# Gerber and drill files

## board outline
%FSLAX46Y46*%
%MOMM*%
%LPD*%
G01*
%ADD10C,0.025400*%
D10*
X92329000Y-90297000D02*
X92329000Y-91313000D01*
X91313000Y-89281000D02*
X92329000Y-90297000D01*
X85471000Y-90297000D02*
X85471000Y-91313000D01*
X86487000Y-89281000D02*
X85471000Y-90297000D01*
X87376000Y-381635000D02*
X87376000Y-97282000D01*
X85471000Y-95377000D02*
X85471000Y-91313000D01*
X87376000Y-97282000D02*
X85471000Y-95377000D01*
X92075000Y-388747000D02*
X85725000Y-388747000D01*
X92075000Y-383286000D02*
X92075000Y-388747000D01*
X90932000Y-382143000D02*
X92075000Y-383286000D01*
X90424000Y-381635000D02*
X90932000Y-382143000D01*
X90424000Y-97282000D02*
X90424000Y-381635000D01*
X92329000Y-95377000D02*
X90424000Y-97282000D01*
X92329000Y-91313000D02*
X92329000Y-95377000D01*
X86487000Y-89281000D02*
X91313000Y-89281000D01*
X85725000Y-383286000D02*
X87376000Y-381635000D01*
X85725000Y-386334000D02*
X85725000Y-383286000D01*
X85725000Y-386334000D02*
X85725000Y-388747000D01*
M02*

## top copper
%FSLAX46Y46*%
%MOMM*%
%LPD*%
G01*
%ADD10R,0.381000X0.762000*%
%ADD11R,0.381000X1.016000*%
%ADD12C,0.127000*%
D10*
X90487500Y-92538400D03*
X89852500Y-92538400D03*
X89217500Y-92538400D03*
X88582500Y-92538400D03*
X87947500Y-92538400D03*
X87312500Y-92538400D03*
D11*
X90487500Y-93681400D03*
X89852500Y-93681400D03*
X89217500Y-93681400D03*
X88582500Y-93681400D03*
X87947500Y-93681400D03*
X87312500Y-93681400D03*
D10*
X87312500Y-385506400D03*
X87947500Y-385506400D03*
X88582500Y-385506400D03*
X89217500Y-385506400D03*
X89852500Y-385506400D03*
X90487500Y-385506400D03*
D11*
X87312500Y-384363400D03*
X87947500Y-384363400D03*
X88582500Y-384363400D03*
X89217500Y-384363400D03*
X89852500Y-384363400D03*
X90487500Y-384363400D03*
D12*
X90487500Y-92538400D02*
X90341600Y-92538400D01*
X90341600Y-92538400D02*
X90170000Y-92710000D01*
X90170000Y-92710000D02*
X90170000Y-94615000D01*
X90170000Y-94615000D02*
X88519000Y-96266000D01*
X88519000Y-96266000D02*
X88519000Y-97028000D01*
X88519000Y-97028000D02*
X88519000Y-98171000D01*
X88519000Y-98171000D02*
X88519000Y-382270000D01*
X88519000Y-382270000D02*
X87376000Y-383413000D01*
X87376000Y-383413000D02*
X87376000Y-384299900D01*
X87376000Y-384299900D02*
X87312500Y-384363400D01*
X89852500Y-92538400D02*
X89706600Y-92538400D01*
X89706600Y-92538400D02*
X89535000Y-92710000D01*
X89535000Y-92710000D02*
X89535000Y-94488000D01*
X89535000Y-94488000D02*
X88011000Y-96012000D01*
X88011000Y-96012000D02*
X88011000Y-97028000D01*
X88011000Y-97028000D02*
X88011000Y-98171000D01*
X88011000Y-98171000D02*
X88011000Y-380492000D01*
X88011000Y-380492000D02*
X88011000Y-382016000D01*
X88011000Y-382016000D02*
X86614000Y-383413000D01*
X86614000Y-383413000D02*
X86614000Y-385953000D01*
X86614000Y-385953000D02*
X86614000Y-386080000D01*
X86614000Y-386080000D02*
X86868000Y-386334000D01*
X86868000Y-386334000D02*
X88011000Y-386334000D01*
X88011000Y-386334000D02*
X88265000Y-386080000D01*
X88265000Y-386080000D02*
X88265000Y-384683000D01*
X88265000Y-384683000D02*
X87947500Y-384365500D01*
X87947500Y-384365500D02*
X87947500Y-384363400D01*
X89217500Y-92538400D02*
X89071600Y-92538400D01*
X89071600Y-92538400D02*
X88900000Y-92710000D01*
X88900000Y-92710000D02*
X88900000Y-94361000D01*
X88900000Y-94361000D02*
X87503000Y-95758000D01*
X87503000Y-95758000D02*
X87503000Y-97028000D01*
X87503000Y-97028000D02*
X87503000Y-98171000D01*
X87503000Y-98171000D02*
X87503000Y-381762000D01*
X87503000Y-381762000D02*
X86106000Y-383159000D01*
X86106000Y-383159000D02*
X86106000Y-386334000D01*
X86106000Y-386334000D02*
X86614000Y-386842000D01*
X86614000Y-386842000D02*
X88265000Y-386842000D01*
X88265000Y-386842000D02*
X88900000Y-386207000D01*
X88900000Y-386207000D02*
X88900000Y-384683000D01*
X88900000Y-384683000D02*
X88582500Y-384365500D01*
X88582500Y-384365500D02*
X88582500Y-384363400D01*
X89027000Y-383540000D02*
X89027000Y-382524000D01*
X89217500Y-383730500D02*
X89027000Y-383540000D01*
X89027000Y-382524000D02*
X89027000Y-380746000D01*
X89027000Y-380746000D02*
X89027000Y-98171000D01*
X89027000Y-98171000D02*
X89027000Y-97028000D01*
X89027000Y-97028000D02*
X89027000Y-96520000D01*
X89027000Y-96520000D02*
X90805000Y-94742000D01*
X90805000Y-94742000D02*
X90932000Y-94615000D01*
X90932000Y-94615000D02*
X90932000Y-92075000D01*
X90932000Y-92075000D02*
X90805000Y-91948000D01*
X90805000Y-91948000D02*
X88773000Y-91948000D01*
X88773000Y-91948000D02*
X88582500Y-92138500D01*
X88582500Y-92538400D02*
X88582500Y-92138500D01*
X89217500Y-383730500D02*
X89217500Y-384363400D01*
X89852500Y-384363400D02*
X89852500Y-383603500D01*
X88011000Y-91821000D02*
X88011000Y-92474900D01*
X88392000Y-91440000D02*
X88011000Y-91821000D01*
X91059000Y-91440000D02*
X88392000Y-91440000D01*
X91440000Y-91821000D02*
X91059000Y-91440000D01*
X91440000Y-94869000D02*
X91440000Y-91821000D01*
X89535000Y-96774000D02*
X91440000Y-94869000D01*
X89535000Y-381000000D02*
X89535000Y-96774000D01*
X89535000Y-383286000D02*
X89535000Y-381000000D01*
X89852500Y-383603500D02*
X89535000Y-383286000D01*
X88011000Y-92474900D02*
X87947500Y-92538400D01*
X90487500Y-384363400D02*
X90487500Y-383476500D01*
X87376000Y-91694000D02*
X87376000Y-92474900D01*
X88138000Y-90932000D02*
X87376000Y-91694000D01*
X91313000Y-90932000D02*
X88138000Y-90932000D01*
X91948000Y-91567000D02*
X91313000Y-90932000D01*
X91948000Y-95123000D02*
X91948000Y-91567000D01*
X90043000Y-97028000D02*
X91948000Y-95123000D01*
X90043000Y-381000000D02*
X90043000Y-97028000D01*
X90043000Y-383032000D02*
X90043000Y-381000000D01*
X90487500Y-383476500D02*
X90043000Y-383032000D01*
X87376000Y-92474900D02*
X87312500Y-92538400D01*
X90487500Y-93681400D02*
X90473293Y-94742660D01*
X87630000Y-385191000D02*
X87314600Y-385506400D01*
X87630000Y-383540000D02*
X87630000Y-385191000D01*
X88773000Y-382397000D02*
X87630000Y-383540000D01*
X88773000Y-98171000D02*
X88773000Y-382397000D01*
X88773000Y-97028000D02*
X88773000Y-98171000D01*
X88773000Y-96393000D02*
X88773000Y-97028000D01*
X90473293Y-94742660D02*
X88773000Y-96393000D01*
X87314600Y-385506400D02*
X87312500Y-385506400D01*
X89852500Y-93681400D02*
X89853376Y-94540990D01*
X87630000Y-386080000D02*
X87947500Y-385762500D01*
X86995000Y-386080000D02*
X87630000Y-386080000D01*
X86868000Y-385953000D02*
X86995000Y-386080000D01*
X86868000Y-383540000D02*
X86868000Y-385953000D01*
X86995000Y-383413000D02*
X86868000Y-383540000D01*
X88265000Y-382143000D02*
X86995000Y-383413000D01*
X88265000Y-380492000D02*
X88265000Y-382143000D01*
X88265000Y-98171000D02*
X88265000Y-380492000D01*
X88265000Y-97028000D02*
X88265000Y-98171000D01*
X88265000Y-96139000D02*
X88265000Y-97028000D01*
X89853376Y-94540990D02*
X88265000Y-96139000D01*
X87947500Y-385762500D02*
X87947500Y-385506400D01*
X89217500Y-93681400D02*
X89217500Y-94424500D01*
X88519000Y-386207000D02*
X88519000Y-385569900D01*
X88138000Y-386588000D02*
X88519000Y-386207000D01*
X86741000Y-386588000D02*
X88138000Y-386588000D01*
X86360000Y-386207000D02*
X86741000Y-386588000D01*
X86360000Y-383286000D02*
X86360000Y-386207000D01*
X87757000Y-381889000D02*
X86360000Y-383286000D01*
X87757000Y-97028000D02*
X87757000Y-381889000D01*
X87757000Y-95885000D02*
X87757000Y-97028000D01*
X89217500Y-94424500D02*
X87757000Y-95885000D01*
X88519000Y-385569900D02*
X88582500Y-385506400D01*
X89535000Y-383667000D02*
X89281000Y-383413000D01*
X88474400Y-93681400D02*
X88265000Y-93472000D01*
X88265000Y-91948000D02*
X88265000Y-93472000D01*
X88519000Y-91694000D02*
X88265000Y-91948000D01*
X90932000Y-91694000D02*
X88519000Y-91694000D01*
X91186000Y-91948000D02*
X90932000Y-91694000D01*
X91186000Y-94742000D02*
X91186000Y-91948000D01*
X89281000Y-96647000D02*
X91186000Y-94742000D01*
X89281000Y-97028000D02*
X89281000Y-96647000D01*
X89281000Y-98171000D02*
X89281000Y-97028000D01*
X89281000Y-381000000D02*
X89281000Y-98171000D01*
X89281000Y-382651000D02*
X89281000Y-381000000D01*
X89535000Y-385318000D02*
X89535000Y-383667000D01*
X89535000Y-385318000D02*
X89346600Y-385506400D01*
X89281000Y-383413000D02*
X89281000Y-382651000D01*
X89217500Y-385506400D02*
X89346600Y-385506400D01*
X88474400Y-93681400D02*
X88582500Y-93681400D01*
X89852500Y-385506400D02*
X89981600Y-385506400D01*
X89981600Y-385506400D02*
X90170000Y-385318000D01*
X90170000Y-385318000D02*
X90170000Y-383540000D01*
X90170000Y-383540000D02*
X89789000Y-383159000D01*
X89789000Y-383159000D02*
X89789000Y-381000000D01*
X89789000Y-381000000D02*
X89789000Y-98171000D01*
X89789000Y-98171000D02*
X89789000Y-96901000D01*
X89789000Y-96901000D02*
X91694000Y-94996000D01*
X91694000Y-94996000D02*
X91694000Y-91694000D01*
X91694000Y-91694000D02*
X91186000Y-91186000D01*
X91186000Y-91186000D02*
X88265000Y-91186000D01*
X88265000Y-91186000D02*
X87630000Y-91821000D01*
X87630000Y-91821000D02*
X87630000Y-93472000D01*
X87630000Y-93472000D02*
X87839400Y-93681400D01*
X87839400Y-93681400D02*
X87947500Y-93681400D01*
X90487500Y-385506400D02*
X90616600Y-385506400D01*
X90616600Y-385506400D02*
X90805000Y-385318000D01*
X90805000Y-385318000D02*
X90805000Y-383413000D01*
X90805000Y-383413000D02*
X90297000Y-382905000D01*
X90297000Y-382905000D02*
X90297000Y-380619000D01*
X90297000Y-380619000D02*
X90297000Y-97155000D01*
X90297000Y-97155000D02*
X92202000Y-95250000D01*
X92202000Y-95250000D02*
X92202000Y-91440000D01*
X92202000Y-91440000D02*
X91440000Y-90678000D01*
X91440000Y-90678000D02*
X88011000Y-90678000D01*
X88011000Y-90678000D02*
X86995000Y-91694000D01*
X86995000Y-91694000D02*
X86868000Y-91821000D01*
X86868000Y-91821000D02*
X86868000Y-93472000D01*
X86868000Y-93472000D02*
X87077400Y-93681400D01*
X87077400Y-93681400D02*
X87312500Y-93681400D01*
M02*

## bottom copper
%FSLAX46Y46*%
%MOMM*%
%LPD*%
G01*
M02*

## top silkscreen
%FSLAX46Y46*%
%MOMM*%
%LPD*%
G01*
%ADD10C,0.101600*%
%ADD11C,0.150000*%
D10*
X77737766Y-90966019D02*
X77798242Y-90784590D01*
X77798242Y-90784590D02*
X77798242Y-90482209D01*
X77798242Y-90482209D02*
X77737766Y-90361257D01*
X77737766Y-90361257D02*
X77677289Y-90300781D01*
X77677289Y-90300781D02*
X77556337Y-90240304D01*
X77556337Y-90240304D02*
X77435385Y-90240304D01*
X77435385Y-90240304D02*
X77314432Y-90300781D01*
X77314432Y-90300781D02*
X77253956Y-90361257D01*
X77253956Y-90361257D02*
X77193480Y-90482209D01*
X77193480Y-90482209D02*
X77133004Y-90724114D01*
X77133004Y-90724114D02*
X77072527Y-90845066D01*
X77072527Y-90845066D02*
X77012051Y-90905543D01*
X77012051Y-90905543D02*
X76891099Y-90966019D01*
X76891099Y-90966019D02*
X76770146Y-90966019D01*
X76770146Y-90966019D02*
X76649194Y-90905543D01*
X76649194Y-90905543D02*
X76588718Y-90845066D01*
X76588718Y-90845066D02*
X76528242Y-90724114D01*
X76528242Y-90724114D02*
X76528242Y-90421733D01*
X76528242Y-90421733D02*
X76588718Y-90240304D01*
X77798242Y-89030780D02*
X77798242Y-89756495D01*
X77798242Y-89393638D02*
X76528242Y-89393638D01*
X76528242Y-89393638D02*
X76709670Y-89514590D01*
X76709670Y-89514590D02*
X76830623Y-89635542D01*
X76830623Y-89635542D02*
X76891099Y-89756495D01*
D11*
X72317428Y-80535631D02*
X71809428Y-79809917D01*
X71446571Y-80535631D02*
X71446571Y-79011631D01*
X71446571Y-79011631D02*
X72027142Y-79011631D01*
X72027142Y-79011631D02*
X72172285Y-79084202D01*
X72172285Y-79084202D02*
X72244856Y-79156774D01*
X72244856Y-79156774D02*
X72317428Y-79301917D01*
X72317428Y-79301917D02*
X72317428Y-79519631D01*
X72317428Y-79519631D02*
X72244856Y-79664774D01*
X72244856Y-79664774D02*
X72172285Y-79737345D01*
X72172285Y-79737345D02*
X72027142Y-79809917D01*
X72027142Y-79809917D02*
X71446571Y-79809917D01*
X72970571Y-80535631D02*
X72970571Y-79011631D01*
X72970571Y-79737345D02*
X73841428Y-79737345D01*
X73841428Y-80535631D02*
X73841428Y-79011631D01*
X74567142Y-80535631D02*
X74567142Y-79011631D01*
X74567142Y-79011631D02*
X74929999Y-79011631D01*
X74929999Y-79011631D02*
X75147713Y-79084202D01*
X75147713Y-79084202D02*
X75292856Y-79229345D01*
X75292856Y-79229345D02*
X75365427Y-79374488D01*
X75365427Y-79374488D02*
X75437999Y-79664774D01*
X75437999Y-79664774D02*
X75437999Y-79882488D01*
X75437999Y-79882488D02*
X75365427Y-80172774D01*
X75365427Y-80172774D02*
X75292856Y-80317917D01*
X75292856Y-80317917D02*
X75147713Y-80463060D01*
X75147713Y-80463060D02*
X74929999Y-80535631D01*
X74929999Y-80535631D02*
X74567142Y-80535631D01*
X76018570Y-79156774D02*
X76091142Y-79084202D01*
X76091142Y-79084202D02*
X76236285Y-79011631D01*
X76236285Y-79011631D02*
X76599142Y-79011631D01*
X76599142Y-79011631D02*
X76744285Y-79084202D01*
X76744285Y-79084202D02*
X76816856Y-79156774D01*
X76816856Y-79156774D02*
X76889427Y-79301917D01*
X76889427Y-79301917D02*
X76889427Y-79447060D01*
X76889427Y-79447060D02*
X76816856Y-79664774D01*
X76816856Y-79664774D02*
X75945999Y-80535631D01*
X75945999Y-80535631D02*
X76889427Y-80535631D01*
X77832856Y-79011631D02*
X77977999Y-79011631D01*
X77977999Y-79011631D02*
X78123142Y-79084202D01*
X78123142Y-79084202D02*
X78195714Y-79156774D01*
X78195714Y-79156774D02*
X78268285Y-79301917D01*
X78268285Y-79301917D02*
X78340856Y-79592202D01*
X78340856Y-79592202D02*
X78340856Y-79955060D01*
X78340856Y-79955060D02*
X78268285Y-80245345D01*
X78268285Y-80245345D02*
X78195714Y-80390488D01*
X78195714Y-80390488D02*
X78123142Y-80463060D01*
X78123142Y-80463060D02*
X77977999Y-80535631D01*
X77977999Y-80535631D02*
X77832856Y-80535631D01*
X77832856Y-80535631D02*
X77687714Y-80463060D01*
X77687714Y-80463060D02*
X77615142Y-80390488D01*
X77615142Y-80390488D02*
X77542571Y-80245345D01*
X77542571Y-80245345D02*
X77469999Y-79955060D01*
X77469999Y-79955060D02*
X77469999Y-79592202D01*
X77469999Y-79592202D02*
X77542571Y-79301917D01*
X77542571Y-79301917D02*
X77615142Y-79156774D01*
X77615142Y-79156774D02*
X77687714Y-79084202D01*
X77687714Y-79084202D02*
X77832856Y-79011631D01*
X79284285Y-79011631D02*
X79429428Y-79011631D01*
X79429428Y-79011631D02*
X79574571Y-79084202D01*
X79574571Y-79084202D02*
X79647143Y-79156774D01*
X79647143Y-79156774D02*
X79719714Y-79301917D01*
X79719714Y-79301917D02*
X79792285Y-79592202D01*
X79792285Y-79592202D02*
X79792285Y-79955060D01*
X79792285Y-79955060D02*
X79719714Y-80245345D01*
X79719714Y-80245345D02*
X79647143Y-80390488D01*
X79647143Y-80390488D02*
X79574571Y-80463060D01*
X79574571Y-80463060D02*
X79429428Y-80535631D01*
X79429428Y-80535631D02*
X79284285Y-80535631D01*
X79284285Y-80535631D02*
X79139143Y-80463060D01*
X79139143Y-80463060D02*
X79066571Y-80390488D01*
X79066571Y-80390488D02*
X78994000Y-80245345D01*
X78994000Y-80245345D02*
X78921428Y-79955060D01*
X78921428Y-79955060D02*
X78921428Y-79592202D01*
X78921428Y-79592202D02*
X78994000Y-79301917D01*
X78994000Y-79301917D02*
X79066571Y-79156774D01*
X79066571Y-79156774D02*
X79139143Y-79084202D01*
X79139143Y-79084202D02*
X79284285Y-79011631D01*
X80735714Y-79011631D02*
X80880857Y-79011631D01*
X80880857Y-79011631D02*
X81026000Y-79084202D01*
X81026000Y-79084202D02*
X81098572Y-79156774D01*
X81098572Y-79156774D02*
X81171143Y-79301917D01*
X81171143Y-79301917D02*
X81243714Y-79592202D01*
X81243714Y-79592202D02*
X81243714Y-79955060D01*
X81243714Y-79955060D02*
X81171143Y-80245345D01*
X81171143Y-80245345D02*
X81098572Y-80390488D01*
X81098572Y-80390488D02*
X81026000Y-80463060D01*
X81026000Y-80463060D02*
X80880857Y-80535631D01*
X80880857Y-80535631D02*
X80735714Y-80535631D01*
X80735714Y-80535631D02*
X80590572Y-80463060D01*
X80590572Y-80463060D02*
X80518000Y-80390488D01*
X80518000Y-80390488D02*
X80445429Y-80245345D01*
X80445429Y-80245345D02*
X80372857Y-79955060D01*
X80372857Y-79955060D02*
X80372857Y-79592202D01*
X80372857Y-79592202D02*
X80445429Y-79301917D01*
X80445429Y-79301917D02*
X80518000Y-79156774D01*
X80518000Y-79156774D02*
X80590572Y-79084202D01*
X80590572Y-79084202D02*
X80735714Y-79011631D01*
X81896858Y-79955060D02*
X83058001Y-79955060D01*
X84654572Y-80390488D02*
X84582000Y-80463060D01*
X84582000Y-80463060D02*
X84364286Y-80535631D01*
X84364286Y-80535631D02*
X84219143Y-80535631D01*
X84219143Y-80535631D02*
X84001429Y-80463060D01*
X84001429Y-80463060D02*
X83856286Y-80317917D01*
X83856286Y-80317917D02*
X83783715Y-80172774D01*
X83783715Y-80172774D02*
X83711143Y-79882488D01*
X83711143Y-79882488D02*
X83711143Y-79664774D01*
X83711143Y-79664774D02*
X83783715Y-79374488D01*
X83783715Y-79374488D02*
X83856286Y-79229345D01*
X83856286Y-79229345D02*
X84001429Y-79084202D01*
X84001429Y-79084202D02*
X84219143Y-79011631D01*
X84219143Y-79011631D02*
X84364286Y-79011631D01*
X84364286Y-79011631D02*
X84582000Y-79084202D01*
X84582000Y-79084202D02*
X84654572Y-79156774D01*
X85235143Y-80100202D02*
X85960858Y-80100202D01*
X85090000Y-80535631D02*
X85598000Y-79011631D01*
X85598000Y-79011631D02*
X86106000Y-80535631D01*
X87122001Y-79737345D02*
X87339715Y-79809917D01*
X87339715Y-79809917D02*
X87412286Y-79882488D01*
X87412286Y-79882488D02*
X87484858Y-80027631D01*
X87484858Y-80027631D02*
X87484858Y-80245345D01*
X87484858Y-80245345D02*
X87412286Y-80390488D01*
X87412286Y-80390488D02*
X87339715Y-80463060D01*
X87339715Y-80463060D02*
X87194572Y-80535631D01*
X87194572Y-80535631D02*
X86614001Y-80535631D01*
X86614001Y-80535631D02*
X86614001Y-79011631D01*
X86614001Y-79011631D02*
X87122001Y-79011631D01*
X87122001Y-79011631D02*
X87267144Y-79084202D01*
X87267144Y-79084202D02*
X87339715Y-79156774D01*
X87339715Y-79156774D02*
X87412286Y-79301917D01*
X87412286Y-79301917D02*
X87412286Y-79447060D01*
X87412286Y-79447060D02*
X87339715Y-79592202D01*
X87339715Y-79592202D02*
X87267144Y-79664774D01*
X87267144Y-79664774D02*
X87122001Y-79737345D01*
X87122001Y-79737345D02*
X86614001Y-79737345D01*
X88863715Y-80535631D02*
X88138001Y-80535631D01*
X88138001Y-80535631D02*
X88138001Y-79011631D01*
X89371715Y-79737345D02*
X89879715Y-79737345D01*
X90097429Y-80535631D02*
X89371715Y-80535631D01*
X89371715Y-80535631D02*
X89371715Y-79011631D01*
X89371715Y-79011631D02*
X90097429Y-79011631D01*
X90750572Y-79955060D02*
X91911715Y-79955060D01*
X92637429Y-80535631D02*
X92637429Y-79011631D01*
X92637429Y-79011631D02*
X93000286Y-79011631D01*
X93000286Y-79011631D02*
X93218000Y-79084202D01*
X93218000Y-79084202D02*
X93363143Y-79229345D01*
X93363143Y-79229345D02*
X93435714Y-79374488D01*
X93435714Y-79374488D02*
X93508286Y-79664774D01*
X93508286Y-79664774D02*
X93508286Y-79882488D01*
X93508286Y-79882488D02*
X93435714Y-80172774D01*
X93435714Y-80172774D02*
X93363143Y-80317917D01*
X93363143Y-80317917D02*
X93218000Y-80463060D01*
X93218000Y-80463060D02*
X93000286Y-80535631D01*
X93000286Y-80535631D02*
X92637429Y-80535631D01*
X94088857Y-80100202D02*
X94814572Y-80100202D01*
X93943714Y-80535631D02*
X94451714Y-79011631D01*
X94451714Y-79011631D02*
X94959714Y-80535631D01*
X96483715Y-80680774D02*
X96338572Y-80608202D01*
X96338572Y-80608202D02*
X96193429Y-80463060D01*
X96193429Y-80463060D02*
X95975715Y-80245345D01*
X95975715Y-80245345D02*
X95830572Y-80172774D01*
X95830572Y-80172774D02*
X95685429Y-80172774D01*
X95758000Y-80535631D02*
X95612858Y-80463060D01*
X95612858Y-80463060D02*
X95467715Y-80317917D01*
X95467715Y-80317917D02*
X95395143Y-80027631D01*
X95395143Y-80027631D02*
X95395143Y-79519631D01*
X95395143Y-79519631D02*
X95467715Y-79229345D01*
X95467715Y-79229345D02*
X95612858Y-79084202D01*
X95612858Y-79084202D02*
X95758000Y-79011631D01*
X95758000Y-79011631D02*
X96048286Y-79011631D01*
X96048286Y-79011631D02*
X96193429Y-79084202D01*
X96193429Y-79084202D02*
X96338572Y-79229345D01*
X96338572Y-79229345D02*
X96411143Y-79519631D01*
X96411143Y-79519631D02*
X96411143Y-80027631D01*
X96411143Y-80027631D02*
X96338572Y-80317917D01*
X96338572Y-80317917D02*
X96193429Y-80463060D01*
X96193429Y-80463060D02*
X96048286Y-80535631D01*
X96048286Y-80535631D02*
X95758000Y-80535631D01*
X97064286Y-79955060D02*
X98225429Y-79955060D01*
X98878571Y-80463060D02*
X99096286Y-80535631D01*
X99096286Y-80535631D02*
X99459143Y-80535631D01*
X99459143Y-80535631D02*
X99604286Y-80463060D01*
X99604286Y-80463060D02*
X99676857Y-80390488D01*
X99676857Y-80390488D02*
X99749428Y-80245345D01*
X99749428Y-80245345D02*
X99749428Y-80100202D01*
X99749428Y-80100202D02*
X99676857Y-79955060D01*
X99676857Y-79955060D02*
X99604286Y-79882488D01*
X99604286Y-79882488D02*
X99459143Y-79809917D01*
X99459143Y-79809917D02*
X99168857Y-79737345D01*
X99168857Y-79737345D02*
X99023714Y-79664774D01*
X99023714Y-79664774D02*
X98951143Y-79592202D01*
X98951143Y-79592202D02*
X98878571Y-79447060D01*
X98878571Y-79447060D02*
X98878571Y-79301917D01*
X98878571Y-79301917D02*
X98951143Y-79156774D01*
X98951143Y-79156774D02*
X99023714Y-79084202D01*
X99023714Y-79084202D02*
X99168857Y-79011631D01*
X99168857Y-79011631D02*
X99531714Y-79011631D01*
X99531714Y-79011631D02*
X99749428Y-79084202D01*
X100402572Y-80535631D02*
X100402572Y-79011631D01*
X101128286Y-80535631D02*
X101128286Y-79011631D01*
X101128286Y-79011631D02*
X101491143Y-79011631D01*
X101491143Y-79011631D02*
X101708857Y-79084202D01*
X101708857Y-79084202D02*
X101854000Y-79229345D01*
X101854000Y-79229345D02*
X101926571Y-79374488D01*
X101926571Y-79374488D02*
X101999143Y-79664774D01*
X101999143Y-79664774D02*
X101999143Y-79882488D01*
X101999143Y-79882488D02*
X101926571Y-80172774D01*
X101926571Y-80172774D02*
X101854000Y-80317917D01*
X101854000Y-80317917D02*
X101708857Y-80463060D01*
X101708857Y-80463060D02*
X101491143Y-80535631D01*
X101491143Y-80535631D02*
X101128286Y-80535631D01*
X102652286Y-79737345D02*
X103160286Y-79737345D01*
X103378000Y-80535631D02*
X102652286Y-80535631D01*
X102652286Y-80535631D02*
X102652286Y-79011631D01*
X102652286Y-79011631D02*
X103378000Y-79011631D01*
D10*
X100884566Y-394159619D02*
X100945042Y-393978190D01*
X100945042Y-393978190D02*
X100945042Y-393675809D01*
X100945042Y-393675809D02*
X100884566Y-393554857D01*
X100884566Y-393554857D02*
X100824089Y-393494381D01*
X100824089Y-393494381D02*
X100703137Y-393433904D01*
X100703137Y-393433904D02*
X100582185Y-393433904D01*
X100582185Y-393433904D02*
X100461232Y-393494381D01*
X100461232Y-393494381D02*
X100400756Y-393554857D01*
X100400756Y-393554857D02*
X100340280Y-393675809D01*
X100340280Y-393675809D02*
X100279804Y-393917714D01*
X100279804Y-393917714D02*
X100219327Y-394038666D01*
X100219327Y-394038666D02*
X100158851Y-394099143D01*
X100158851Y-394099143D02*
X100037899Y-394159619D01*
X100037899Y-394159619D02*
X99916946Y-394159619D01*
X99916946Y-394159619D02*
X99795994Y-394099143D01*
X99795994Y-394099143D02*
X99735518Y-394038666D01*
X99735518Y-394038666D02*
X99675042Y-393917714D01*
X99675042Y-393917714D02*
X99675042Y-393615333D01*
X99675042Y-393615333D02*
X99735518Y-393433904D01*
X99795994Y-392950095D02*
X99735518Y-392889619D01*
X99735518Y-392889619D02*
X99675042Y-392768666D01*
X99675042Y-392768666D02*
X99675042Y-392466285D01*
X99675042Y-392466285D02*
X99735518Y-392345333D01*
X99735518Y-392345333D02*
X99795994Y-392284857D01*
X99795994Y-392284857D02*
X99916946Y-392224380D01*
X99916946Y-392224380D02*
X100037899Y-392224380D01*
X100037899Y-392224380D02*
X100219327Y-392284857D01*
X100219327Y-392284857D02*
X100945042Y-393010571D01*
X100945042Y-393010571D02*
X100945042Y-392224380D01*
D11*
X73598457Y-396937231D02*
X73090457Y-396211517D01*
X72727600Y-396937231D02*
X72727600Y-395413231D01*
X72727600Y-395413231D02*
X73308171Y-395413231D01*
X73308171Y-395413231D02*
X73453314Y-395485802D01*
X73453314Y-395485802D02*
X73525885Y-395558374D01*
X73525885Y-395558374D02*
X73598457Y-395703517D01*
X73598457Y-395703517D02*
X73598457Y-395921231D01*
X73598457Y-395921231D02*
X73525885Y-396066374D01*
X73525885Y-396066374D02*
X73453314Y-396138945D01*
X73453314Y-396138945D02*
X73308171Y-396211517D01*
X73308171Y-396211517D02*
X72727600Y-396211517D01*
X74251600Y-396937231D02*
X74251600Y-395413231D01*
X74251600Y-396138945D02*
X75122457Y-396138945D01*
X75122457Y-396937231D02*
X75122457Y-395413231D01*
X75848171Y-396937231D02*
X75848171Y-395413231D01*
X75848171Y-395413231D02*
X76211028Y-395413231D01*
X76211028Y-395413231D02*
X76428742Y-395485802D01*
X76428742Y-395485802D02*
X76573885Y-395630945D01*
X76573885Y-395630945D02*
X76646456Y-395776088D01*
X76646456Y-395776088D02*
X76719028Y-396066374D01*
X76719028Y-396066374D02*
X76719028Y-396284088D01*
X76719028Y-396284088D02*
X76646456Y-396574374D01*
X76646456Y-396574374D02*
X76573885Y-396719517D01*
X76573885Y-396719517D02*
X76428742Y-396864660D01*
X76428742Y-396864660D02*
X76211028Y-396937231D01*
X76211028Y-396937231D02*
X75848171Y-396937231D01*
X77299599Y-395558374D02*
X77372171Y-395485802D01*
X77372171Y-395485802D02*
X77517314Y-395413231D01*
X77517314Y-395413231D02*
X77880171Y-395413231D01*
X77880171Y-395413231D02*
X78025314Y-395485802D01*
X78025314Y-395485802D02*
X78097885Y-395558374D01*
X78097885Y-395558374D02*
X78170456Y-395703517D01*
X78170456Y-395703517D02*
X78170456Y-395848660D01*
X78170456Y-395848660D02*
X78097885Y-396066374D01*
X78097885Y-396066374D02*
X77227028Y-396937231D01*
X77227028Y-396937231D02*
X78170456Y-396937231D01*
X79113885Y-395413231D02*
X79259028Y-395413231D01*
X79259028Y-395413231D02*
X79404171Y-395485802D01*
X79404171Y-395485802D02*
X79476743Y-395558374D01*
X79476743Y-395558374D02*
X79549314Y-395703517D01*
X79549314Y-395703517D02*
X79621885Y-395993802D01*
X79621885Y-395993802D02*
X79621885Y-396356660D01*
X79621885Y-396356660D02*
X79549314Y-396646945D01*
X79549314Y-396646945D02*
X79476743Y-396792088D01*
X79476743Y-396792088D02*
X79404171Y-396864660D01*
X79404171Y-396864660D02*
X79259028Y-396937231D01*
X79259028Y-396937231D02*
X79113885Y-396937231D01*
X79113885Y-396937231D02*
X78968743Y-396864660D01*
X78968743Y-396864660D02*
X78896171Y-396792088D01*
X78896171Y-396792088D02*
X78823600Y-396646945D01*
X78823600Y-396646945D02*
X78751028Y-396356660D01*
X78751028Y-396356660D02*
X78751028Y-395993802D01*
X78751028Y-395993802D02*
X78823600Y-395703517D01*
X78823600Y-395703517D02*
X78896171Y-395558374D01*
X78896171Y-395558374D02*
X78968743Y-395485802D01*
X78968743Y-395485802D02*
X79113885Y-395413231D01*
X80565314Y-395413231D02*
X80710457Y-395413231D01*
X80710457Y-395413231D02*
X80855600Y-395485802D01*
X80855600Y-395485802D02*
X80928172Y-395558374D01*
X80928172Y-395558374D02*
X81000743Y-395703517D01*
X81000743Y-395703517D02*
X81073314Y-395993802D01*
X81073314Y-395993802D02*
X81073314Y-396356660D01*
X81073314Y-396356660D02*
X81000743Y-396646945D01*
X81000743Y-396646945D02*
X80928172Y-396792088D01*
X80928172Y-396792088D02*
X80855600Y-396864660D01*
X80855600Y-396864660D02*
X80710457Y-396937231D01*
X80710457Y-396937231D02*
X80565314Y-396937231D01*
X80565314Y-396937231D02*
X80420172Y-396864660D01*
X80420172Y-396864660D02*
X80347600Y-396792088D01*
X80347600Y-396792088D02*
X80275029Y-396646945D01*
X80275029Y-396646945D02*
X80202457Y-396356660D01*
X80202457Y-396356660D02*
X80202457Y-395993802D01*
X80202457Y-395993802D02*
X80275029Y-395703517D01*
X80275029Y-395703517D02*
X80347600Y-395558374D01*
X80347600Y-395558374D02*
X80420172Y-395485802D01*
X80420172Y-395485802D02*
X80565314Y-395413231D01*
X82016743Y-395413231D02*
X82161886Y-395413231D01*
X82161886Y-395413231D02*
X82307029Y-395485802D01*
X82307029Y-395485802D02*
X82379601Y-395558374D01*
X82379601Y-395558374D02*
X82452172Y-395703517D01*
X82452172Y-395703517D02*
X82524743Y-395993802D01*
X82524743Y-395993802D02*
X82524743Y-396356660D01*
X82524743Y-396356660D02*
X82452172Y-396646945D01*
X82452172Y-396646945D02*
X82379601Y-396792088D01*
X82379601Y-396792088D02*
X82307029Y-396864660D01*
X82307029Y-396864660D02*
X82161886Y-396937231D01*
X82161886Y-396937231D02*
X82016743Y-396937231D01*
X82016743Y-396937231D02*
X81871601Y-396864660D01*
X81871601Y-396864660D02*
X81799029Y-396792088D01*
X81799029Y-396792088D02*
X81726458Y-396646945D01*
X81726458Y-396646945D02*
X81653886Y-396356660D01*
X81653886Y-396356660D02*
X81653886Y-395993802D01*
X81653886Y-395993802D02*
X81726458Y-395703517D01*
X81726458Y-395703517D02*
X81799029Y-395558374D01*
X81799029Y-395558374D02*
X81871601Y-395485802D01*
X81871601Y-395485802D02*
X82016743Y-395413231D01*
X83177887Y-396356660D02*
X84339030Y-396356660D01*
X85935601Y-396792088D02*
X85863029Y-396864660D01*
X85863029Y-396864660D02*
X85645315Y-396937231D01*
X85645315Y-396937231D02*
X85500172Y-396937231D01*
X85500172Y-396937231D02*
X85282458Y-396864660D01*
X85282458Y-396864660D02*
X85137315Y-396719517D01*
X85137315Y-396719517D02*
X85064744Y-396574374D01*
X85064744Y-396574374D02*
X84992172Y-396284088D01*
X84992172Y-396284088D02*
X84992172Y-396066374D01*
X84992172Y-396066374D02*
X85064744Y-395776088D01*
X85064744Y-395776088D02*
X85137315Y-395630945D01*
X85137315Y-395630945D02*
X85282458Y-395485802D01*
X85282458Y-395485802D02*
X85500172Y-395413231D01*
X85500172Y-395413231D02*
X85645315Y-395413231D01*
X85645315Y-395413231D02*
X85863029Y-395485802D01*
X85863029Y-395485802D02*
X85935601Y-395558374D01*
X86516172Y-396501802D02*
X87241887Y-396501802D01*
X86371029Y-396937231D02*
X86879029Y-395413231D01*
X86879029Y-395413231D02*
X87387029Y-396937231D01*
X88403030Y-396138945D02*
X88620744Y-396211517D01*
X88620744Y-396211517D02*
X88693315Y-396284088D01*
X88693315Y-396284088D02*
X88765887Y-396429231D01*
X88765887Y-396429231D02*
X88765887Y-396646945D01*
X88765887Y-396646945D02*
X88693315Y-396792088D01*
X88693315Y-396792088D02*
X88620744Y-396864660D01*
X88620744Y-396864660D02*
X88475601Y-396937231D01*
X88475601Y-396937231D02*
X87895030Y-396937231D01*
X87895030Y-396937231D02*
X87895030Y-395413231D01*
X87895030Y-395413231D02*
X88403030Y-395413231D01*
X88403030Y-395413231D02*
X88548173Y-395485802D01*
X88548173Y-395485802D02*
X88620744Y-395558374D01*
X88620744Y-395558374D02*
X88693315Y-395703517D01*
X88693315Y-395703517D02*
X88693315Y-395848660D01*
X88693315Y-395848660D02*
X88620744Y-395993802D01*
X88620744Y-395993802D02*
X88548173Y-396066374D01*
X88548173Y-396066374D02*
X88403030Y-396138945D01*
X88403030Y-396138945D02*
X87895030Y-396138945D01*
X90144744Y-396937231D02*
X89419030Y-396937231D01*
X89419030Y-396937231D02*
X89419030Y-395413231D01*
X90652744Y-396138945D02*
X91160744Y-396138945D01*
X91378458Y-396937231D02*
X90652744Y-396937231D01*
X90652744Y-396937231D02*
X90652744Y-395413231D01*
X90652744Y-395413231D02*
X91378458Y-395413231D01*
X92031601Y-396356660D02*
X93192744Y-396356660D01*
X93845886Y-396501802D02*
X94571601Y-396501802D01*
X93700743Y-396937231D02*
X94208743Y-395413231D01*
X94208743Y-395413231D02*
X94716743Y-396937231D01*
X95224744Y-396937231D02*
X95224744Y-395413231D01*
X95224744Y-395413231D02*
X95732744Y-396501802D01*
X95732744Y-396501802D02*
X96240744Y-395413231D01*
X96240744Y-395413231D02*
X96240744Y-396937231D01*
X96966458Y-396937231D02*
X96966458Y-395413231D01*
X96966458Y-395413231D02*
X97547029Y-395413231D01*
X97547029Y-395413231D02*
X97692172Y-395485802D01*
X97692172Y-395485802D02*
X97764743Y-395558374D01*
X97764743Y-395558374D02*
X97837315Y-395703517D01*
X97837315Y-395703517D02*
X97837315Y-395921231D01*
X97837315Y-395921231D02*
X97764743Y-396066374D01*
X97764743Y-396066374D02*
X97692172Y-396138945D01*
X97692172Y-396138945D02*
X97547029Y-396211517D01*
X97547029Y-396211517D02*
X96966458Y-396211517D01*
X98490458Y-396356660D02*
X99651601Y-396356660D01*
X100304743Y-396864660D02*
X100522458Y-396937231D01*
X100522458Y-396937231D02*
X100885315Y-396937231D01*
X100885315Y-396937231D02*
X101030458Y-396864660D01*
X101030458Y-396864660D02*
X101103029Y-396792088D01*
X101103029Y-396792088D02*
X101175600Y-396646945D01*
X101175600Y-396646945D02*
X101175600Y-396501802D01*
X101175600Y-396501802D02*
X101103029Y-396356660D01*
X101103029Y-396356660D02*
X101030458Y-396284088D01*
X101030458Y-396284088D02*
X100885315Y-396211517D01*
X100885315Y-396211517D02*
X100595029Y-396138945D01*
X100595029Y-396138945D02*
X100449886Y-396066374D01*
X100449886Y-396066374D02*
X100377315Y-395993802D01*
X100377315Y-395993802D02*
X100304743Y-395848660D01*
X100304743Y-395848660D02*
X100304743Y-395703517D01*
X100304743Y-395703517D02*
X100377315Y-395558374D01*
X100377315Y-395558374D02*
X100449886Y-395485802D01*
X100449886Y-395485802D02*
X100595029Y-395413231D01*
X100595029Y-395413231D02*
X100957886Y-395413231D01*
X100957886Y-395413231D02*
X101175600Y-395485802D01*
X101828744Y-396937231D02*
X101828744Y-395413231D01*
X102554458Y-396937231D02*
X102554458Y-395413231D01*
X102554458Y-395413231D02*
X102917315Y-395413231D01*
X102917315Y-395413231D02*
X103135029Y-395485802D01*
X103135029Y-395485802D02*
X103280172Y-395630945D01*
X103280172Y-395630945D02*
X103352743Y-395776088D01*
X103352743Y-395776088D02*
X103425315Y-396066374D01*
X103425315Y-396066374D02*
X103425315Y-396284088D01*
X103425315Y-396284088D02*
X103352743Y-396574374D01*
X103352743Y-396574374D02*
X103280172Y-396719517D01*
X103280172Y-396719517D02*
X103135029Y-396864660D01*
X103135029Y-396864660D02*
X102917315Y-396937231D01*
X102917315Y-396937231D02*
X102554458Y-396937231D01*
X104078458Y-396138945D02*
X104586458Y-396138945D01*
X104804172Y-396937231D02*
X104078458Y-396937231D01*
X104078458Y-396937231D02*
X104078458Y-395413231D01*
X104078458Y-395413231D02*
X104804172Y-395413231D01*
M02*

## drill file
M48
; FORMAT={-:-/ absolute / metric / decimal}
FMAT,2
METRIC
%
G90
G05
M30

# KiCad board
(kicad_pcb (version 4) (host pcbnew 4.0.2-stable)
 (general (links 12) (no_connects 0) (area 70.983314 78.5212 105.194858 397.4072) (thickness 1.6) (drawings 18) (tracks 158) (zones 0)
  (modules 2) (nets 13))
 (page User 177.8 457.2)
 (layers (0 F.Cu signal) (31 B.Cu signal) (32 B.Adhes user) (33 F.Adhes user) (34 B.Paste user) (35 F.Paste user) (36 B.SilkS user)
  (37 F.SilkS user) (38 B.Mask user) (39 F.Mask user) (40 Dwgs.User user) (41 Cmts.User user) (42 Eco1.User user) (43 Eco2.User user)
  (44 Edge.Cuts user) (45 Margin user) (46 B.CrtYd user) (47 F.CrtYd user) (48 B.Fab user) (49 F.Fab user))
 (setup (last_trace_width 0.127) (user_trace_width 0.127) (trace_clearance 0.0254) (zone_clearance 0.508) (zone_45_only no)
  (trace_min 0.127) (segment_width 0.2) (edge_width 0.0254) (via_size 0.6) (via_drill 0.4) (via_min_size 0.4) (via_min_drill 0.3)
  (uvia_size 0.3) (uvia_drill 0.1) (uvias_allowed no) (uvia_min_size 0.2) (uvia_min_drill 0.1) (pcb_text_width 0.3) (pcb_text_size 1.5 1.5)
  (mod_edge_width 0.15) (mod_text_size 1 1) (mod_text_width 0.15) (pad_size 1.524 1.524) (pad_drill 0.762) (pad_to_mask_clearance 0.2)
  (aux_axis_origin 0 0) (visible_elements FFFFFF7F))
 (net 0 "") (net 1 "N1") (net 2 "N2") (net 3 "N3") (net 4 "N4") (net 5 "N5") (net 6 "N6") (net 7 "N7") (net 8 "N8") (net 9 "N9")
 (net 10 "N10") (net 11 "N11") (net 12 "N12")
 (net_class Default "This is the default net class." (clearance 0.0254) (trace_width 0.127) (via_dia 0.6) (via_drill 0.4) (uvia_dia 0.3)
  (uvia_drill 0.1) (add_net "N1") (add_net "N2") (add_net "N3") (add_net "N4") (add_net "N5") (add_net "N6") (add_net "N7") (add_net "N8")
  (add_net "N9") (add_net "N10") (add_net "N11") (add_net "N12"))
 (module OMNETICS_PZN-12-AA (layer F.Cu) (at 88.9 91.5224)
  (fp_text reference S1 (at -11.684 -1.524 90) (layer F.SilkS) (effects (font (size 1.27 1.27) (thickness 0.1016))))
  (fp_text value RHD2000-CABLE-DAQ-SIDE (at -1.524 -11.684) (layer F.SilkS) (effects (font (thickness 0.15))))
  (pad B1 smd rect (at 1.5875 1.016 180) (size 0.381 0.762) (layers F.Cu F.Paste F.Mask) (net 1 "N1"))
  (pad B2 smd rect (at 0.9525 1.016 180) (size 0.381 0.762) (layers F.Cu F.Paste F.Mask) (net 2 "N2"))
  (pad B3 smd rect (at 0.3175 1.016 180) (size 0.381 0.762) (layers F.Cu F.Paste F.Mask) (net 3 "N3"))
  (pad B4 smd rect (at -0.3175 1.016 180) (size 0.381 0.762) (layers F.Cu F.Paste F.Mask) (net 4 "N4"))
  (pad B5 smd rect (at -0.9525 1.016 180) (size 0.381 0.762) (layers F.Cu F.Paste F.Mask) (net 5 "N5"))
  (pad B6 smd rect (at -1.5875 1.016 180) (size 0.381 0.762) (layers F.Cu F.Paste F.Mask) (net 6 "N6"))
  (pad T1 smd rect (at 1.5875 2.159 180) (size 0.381 1.016) (layers F.Cu F.Paste F.Mask) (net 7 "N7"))
  (pad T2 smd rect (at 0.9525 2.159 180) (size 0.381 1.016) (layers F.Cu F.Paste F.Mask) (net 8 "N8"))
  (pad T3 smd rect (at 0.3175 2.159 180) (size 0.381 1.016) (layers F.Cu F.Paste F.Mask) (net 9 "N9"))
  (pad T4 smd rect (at -0.3175 2.159 180) (size 0.381 1.016) (layers F.Cu F.Paste F.Mask) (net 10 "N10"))
  (pad T5 smd rect (at -0.9525 2.159 180) (size 0.381 1.016) (layers F.Cu F.Paste F.Mask) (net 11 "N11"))
  (pad T6 smd rect (at -1.5875 2.159 180) (size 0.381 1.016) (layers F.Cu F.Paste F.Mask) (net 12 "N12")))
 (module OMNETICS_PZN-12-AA (layer F.Cu) (at 88.9 386.5224 180)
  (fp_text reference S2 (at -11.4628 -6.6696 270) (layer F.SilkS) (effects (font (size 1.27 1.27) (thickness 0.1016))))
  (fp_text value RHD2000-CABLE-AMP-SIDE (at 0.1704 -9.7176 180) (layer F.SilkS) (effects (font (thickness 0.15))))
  (pad B1 smd rect (at 1.5875 1.016) (size 0.381 0.762) (layers F.Cu F.Paste F.Mask) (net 7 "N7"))
  (pad B2 smd rect (at 0.9525 1.016) (size 0.381 0.762) (layers F.Cu F.Paste F.Mask) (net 8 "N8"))
  (pad B3 smd rect (at 0.3175 1.016) (size 0.381 0.762) (layers F.Cu F.Paste F.Mask) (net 9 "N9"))
  (pad B4 smd rect (at -0.3175 1.016) (size 0.381 0.762) (layers F.Cu F.Paste F.Mask) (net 10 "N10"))
  (pad B5 smd rect (at -0.9525 1.016) (size 0.381 0.762) (layers F.Cu F.Paste F.Mask) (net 11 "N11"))
  (pad B6 smd rect (at -1.5875 1.016) (size 0.381 0.762) (layers F.Cu F.Paste F.Mask) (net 12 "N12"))
  (pad T1 smd rect (at 1.5875 2.159) (size 0.381 1.016) (layers F.Cu F.Paste F.Mask) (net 1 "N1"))
  (pad T2 smd rect (at 0.9525 2.159) (size 0.381 1.016) (layers F.Cu F.Paste F.Mask) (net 2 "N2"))
  (pad T3 smd rect (at 0.3175 2.159) (size 0.381 1.016) (layers F.Cu F.Paste F.Mask) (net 3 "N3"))
  (pad T4 smd rect (at -0.3175 2.159) (size 0.381 1.016) (layers F.Cu F.Paste F.Mask) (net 4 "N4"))
  (pad T5 smd rect (at -0.9525 2.159) (size 0.381 1.016) (layers F.Cu F.Paste F.Mask) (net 5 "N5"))
  (pad T6 smd rect (at -1.5875 2.159) (size 0.381 1.016) (layers F.Cu F.Paste F.Mask) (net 6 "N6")))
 (gr_line (start 92.329 90.297) (end 92.329 91.313) (angle 90) (layer Edge.Cuts) (width 0.0254))
 (gr_line (start 91.313 89.281) (end 92.329 90.297) (angle 90) (layer Edge.Cuts) (width 0.0254))
 (gr_line (start 85.471 90.297) (end 85.471 91.313) (angle 90) (layer Edge.Cuts) (width 0.0254))
 (gr_line (start 86.487 89.281) (end 85.471 90.297) (angle 90) (layer Edge.Cuts) (width 0.0254))
 (gr_line (start 87.376 381.635) (end 87.376 97.282) (angle 90) (layer Edge.Cuts) (width 0.0254))
 (gr_line (start 85.471 95.377) (end 85.471 91.313) (angle 90) (layer Edge.Cuts) (width 0.0254))
 (gr_line (start 87.376 97.282) (end 85.471 95.377) (angle 90) (layer Edge.Cuts) (width 0.0254))
 (gr_line (start 92.075 388.747) (end 85.725 388.747) (angle 90) (layer Edge.Cuts) (width 0.0254))
 (gr_line (start 92.075 383.286) (end 92.075 388.747) (angle 90) (layer Edge.Cuts) (width 0.0254))
 (gr_line (start 90.932 382.143) (end 92.075 383.286) (angle 90) (layer Edge.Cuts) (width 0.0254))
 (gr_line (start 90.424 381.635) (end 90.932 382.143) (angle 90) (layer Edge.Cuts) (width 0.0254))
 (gr_line (start 90.424 97.282) (end 90.424 381.635) (angle 90) (layer Edge.Cuts) (width 0.0254))
 (gr_line (start 92.329 95.377) (end 90.424 97.282) (angle 90) (layer Edge.Cuts) (width 0.0254))
 (gr_line (start 92.329 91.313) (end 92.329 95.377) (angle 90) (layer Edge.Cuts) (width 0.0254))
 (gr_line (start 86.487 89.281) (end 91.313 89.281) (angle 90) (layer Edge.Cuts) (width 0.0254))
 (gr_line (start 85.725 383.286) (end 87.376 381.635) (angle 90) (layer Edge.Cuts) (width 0.0254))
 (gr_line (start 85.725 386.334) (end 85.725 383.286) (angle 90) (layer Edge.Cuts) (width 0.0254))
 (gr_line (start 85.725 386.334) (end 85.725 388.747) (angle 90) (layer Edge.Cuts) (width 0.0254))
 (segment (start 90.4875 92.5384) (end 90.3416 92.5384) (width 0.127) (layer F.Cu) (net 1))
 (segment (start 90.3416 92.5384) (end 90.17 92.71) (width 0.127) (layer F.Cu) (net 1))
 (segment (start 90.17 92.71) (end 90.17 94.615) (width 0.127) (layer F.Cu) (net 1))
 (segment (start 90.17 94.615) (end 88.519 96.266) (width 0.127) (layer F.Cu) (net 1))
 (segment (start 88.519 96.266) (end 88.519 97.028) (width 0.127) (layer F.Cu) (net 1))
 (segment (start 88.519 97.028) (end 88.519 98.171) (width 0.127) (layer F.Cu) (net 1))
 (segment (start 88.519 98.171) (end 88.519 382.27) (width 0.127) (layer F.Cu) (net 1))
 (segment (start 88.519 382.27) (end 87.376 383.413) (width 0.127) (layer F.Cu) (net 1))
 (segment (start 87.376 383.413) (end 87.376 384.2999) (width 0.127) (layer F.Cu) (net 1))
 (segment (start 87.376 384.2999) (end 87.3125 384.3634) (width 0.127) (layer F.Cu) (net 1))
 (segment (start 89.8525 92.5384) (end 89.7066 92.5384) (width 0.127) (layer F.Cu) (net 2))
 (segment (start 89.7066 92.5384) (end 89.535 92.71) (width 0.127) (layer F.Cu) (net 2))
 (segment (start 89.535 92.71) (end 89.535 94.488) (width 0.127) (layer F.Cu) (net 2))
 (segment (start 89.535 94.488) (end 88.011 96.012) (width 0.127) (layer F.Cu) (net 2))
 (segment (start 88.011 96.012) (end 88.011 97.028) (width 0.127) (layer F.Cu) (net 2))
 (segment (start 88.011 97.028) (end 88.011 98.171) (width 0.127) (layer F.Cu) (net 2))
 (segment (start 88.011 98.171) (end 88.011 380.492) (width 0.127) (layer F.Cu) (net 2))
 (segment (start 88.011 380.492) (end 88.011 382.016) (width 0.127) (layer F.Cu) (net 2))
 (segment (start 88.011 382.016) (end 86.614 383.413) (width 0.127) (layer F.Cu) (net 2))
 (segment (start 86.614 383.413) (end 86.614 385.953) (width 0.127) (layer F.Cu) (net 2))
 (segment (start 86.614 385.953) (end 86.614 386.08) (width 0.127) (layer F.Cu) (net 2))
 (segment (start 86.614 386.08) (end 86.868 386.334) (width 0.127) (layer F.Cu) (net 2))
 (segment (start 86.868 386.334) (end 88.011 386.334) (width 0.127) (layer F.Cu) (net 2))
 (segment (start 88.011 386.334) (end 88.265 386.08) (width 0.127) (layer F.Cu) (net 2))
 (segment (start 88.265 386.08) (end 88.265 384.683) (width 0.127) (layer F.Cu) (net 2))
 (segment (start 88.265 384.683) (end 87.9475 384.3655) (width 0.127) (layer F.Cu) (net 2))
 (segment (start 87.9475 384.3655) (end 87.9475 384.3634) (width 0.127) (layer F.Cu) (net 2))
 (segment (start 89.2175 92.5384) (end 89.0716 92.5384) (width 0.127) (layer F.Cu) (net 3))
 (segment (start 89.0716 92.5384) (end 88.9 92.71) (width 0.127) (layer F.Cu) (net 3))
 (segment (start 88.9 92.71) (end 88.9 94.361) (width 0.127) (layer F.Cu) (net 3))
 (segment (start 88.9 94.361) (end 87.503 95.758) (width 0.127) (layer F.Cu) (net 3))
 (segment (start 87.503 95.758) (end 87.503 97.028) (width 0.127) (layer F.Cu) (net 3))
 (segment (start 87.503 97.028) (end 87.503 98.171) (width 0.127) (layer F.Cu) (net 3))
 (segment (start 87.503 98.171) (end 87.503 381.762) (width 0.127) (layer F.Cu) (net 3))
 (segment (start 87.503 381.762) (end 86.106 383.159) (width 0.127) (layer F.Cu) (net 3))
 (segment (start 86.106 383.159) (end 86.106 386.334) (width 0.127) (layer F.Cu) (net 3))
 (segment (start 86.106 386.334) (end 86.614 386.842) (width 0.127) (layer F.Cu) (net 3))
 (segment (start 86.614 386.842) (end 88.265 386.842) (width 0.127) (layer F.Cu) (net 3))
 (segment (start 88.265 386.842) (end 88.9 386.207) (width 0.127) (layer F.Cu) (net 3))
 (segment (start 88.9 386.207) (end 88.9 384.683) (width 0.127) (layer F.Cu) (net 3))
 (segment (start 88.9 384.683) (end 88.5825 384.3655) (width 0.127) (layer F.Cu) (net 3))
 (segment (start 88.5825 384.3655) (end 88.5825 384.3634) (width 0.127) (layer F.Cu) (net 3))
 (segment (start 89.027 383.54) (end 89.027 382.524) (width 0.127) (layer F.Cu) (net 4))
 (segment (start 89.2175 383.7305) (end 89.027 383.54) (width 0.127) (layer F.Cu) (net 4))
 (segment (start 89.027 382.524) (end 89.027 380.746) (width 0.127) (layer F.Cu) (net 4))
 (segment (start 89.027 380.746) (end 89.027 98.171) (width 0.127) (layer F.Cu) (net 4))
 (segment (start 89.027 98.171) (end 89.027 97.028) (width 0.127) (layer F.Cu) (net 4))
 (segment (start 89.027 97.028) (end 89.027 96.52) (width 0.127) (layer F.Cu) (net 4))
 (segment (start 89.027 96.52) (end 90.805 94.742) (width 0.127) (layer F.Cu) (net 4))
 (segment (start 90.805 94.742) (end 90.932 94.615) (width 0.127) (layer F.Cu) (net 4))
 (segment (start 90.932 94.615) (end 90.932 92.075) (width 0.127) (layer F.Cu) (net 4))
 (segment (start 90.932 92.075) (end 90.805 91.948) (width 0.127) (layer F.Cu) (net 4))
 (segment (start 90.805 91.948) (end 88.773 91.948) (width 0.127) (layer F.Cu) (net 4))
 (segment (start 88.773 91.948) (end 88.5825 92.1385) (width 0.127) (layer F.Cu) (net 4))
 (segment (start 88.5825 92.5384) (end 88.5825 92.1385) (width 0.127) (layer F.Cu) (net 4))
 (segment (start 89.2175 383.7305) (end 89.2175 384.3634) (width 0.127) (layer F.Cu) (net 4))
 (segment (start 89.8525 384.3634) (end 89.8525 383.6035) (width 0.127) (layer F.Cu) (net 5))
 (segment (start 88.011 91.821) (end 88.011 92.4749) (width 0.127) (layer F.Cu) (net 5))
 (segment (start 88.392 91.44) (end 88.011 91.821) (width 0.127) (layer F.Cu) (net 5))
 (segment (start 91.059 91.44) (end 88.392 91.44) (width 0.127) (layer F.Cu) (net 5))
 (segment (start 91.44 91.821) (end 91.059 91.44) (width 0.127) (layer F.Cu) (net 5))
 (segment (start 91.44 94.869) (end 91.44 91.821) (width 0.127) (layer F.Cu) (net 5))
 (segment (start 89.535 96.774) (end 91.44 94.869) (width 0.127) (layer F.Cu) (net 5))
 (segment (start 89.535 381) (end 89.535 96.774) (width 0.127) (layer F.Cu) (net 5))
 (segment (start 89.535 383.286) (end 89.535 381) (width 0.127) (layer F.Cu) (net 5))
 (segment (start 89.8525 383.6035) (end 89.535 383.286) (width 0.127) (layer F.Cu) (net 5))
 (segment (start 88.011 92.4749) (end 87.9475 92.5384) (width 0.127) (layer F.Cu) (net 5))
 (segment (start 90.4875 384.3634) (end 90.4875 383.4765) (width 0.127) (layer F.Cu) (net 6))
 (segment (start 87.376 91.694) (end 87.376 92.4749) (width 0.127) (layer F.Cu) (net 6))
 (segment (start 88.138 90.932) (end 87.376 91.694) (width 0.127) (layer F.Cu) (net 6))
 (segment (start 91.313 90.932) (end 88.138 90.932) (width 0.127) (layer F.Cu) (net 6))
 (segment (start 91.948 91.567) (end 91.313 90.932) (width 0.127) (layer F.Cu) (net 6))
 (segment (start 91.948 95.123) (end 91.948 91.567) (width 0.127) (layer F.Cu) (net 6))
 (segment (start 90.043 97.028) (end 91.948 95.123) (width 0.127) (layer F.Cu) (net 6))
 (segment (start 90.043 381) (end 90.043 97.028) (width 0.127) (layer F.Cu) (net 6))
 (segment (start 90.043 383.032) (end 90.043 381) (width 0.127) (layer F.Cu) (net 6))
 (segment (start 90.4875 383.4765) (end 90.043 383.032) (width 0.127) (layer F.Cu) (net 6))
 (segment (start 87.376 92.4749) (end 87.3125 92.5384) (width 0.127) (layer F.Cu) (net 6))
 (segment (start 90.4875 93.6814) (end 90.473293 94.74266) (width 0.127) (layer F.Cu) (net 7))
 (segment (start 87.63 385.191) (end 87.3146 385.5064) (width 0.127) (layer F.Cu) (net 7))
 (segment (start 87.63 383.54) (end 87.63 385.191) (width 0.127) (layer F.Cu) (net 7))
 (segment (start 88.773 382.397) (end 87.63 383.54) (width 0.127) (layer F.Cu) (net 7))
 (segment (start 88.773 98.171) (end 88.773 382.397) (width 0.127) (layer F.Cu) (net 7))
 (segment (start 88.773 97.028) (end 88.773 98.171) (width 0.127) (layer F.Cu) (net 7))
 (segment (start 88.773 96.393) (end 88.773 97.028) (width 0.127) (layer F.Cu) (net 7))
 (segment (start 90.473293 94.74266) (end 88.773 96.393) (width 0.127) (layer F.Cu) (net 7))
 (segment (start 87.3146 385.5064) (end 87.3125 385.5064) (width 0.127) (layer F.Cu) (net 7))
 (segment (start 89.8525 93.6814) (end 89.853376 94.54099) (width 0.127) (layer F.Cu) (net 8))
 (segment (start 87.63 386.08) (end 87.9475 385.7625) (width 0.127) (layer F.Cu) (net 8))
 (segment (start 86.995 386.08) (end 87.63 386.08) (width 0.127) (layer F.Cu) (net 8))
 (segment (start 86.868 385.953) (end 86.995 386.08) (width 0.127) (layer F.Cu) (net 8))
 (segment (start 86.868 383.54) (end 86.868 385.953) (width 0.127) (layer F.Cu) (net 8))
 (segment (start 86.995 383.413) (end 86.868 383.54) (width 0.127) (layer F.Cu) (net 8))
 (segment (start 88.265 382.143) (end 86.995 383.413) (width 0.127) (layer F.Cu) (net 8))
 (segment (start 88.265 380.492) (end 88.265 382.143) (width 0.127) (layer F.Cu) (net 8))
 (segment (start 88.265 98.171) (end 88.265 380.492) (width 0.127) (layer F.Cu) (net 8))
 (segment (start 88.265 97.028) (end 88.265 98.171) (width 0.127) (layer F.Cu) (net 8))
 (segment (start 88.265 96.139) (end 88.265 97.028) (width 0.127) (layer F.Cu) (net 8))
 (segment (start 89.853376 94.54099) (end 88.265 96.139) (width 0.127) (layer F.Cu) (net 8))
 (segment (start 87.9475 385.7625) (end 87.9475 385.5064) (width 0.127) (layer F.Cu) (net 8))
 (segment (start 89.2175 93.6814) (end 89.2175 94.4245) (width 0.127) (layer F.Cu) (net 9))
 (segment (start 88.519 386.207) (end 88.519 385.5699) (width 0.127) (layer F.Cu) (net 9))
 (segment (start 88.138 386.588) (end 88.519 386.207) (width 0.127) (layer F.Cu) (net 9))
 (segment (start 86.741 386.588) (end 88.138 386.588) (width 0.127) (layer F.Cu) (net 9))
 (segment (start 86.36 386.207) (end 86.741 386.588) (width 0.127) (layer F.Cu) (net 9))
 (segment (start 86.36 383.286) (end 86.36 386.207) (width 0.127) (layer F.Cu) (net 9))
 (segment (start 87.757 381.889) (end 86.36 383.286) (width 0.127) (layer F.Cu) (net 9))
 (segment (start 87.757 97.028) (end 87.757 381.889) (width 0.127) (layer F.Cu) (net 9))
 (segment (start 87.757 95.885) (end 87.757 97.028) (width 0.127) (layer F.Cu) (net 9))
 (segment (start 89.2175 94.4245) (end 87.757 95.885) (width 0.127) (layer F.Cu) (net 9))
 (segment (start 88.519 385.5699) (end 88.5825 385.5064) (width 0.127) (layer F.Cu) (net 9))
 (segment (start 89.535 383.667) (end 89.281 383.413) (width 0.127) (layer F.Cu) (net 10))
 (segment (start 88.4744 93.6814) (end 88.265 93.472) (width 0.127) (layer F.Cu) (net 10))
 (segment (start 88.265 91.948) (end 88.265 93.472) (width 0.127) (layer F.Cu) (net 10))
 (segment (start 88.519 91.694) (end 88.265 91.948) (width 0.127) (layer F.Cu) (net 10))
 (segment (start 90.932 91.694) (end 88.519 91.694) (width 0.127) (layer F.Cu) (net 10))
 (segment (start 91.186 91.948) (end 90.932 91.694) (width 0.127) (layer F.Cu) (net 10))
 (segment (start 91.186 94.742) (end 91.186 91.948) (width 0.127) (layer F.Cu) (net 10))
 (segment (start 89.281 96.647) (end 91.186 94.742) (width 0.127) (layer F.Cu) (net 10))
 (segment (start 89.281 97.028) (end 89.281 96.647) (width 0.127) (layer F.Cu) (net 10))
 (segment (start 89.281 98.171) (end 89.281 97.028) (width 0.127) (layer F.Cu) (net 10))
 (segment (start 89.281 381) (end 89.281 98.171) (width 0.127) (layer F.Cu) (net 10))
 (segment (start 89.281 382.651) (end 89.281 381) (width 0.127) (layer F.Cu) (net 10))
 (segment (start 89.535 385.318) (end 89.535 383.667) (width 0.127) (layer F.Cu) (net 10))
 (segment (start 89.535 385.318) (end 89.3466 385.5064) (width 0.127) (layer F.Cu) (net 10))
 (segment (start 89.281 383.413) (end 89.281 382.651) (width 0.127) (layer F.Cu) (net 10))
 (segment (start 89.2175 385.5064) (end 89.3466 385.5064) (width 0.127) (layer F.Cu) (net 10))
 (segment (start 88.4744 93.6814) (end 88.5825 93.6814) (width 0.127) (layer F.Cu) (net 10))
 (segment (start 89.8525 385.5064) (end 89.9816 385.5064) (width 0.127) (layer F.Cu) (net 11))
 (segment (start 89.9816 385.5064) (end 90.17 385.318) (width 0.127) (layer F.Cu) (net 11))
 (segment (start 90.17 385.318) (end 90.17 383.54) (width 0.127) (layer F.Cu) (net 11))
 (segment (start 90.17 383.54) (end 89.789 383.159) (width 0.127) (layer F.Cu) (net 11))
 (segment (start 89.789 383.159) (end 89.789 381) (width 0.127) (layer F.Cu) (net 11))
 (segment (start 89.789 381) (end 89.789 98.171) (width 0.127) (layer F.Cu) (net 11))
 (segment (start 89.789 98.171) (end 89.789 96.901) (width 0.127) (layer F.Cu) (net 11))
 (segment (start 89.789 96.901) (end 91.694 94.996) (width 0.127) (layer F.Cu) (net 11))
 (segment (start 91.694 94.996) (end 91.694 91.694) (width 0.127) (layer F.Cu) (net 11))
 (segment (start 91.694 91.694) (end 91.186 91.186) (width 0.127) (layer F.Cu) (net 11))
 (segment (start 91.186 91.186) (end 88.265 91.186) (width 0.127) (layer F.Cu) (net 11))
 (segment (start 88.265 91.186) (end 87.63 91.821) (width 0.127) (layer F.Cu) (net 11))
 (segment (start 87.63 91.821) (end 87.63 93.472) (width 0.127) (layer F.Cu) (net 11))
 (segment (start 87.63 93.472) (end 87.8394 93.6814) (width 0.127) (layer F.Cu) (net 11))
 (segment (start 87.8394 93.6814) (end 87.9475 93.6814) (width 0.127) (layer F.Cu) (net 11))
 (segment (start 90.4875 385.5064) (end 90.6166 385.5064) (width 0.127) (layer F.Cu) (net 12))
 (segment (start 90.6166 385.5064) (end 90.805 385.318) (width 0.127) (layer F.Cu) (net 12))
 (segment (start 90.805 385.318) (end 90.805 383.413) (width 0.127) (layer F.Cu) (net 12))
 (segment (start 90.805 383.413) (end 90.297 382.905) (width 0.127) (layer F.Cu) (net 12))
 (segment (start 90.297 382.905) (end 90.297 380.619) (width 0.127) (layer F.Cu) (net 12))
 (segment (start 90.297 380.619) (end 90.297 97.155) (width 0.127) (layer F.Cu) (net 12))
 (segment (start 90.297 97.155) (end 92.202 95.25) (width 0.127) (layer F.Cu) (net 12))
 (segment (start 92.202 95.25) (end 92.202 91.44) (width 0.127) (layer F.Cu) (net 12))
 (segment (start 92.202 91.44) (end 91.44 90.678) (width 0.127) (layer F.Cu) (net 12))
 (segment (start 91.44 90.678) (end 88.011 90.678) (width 0.127) (layer F.Cu) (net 12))
 (segment (start 88.011 90.678) (end 86.995 91.694) (width 0.127) (layer F.Cu) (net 12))
 (segment (start 86.995 91.694) (end 86.868 91.821) (width 0.127) (layer F.Cu) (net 12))
 (segment (start 86.868 91.821) (end 86.868 93.472) (width 0.127) (layer F.Cu) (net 12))
 (segment (start 86.868 93.472) (end 87.0774 93.6814) (width 0.127) (layer F.Cu) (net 12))
 (segment (start 87.0774 93.6814) (end 87.3125 93.6814) (width 0.127) (layer F.Cu) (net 12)))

